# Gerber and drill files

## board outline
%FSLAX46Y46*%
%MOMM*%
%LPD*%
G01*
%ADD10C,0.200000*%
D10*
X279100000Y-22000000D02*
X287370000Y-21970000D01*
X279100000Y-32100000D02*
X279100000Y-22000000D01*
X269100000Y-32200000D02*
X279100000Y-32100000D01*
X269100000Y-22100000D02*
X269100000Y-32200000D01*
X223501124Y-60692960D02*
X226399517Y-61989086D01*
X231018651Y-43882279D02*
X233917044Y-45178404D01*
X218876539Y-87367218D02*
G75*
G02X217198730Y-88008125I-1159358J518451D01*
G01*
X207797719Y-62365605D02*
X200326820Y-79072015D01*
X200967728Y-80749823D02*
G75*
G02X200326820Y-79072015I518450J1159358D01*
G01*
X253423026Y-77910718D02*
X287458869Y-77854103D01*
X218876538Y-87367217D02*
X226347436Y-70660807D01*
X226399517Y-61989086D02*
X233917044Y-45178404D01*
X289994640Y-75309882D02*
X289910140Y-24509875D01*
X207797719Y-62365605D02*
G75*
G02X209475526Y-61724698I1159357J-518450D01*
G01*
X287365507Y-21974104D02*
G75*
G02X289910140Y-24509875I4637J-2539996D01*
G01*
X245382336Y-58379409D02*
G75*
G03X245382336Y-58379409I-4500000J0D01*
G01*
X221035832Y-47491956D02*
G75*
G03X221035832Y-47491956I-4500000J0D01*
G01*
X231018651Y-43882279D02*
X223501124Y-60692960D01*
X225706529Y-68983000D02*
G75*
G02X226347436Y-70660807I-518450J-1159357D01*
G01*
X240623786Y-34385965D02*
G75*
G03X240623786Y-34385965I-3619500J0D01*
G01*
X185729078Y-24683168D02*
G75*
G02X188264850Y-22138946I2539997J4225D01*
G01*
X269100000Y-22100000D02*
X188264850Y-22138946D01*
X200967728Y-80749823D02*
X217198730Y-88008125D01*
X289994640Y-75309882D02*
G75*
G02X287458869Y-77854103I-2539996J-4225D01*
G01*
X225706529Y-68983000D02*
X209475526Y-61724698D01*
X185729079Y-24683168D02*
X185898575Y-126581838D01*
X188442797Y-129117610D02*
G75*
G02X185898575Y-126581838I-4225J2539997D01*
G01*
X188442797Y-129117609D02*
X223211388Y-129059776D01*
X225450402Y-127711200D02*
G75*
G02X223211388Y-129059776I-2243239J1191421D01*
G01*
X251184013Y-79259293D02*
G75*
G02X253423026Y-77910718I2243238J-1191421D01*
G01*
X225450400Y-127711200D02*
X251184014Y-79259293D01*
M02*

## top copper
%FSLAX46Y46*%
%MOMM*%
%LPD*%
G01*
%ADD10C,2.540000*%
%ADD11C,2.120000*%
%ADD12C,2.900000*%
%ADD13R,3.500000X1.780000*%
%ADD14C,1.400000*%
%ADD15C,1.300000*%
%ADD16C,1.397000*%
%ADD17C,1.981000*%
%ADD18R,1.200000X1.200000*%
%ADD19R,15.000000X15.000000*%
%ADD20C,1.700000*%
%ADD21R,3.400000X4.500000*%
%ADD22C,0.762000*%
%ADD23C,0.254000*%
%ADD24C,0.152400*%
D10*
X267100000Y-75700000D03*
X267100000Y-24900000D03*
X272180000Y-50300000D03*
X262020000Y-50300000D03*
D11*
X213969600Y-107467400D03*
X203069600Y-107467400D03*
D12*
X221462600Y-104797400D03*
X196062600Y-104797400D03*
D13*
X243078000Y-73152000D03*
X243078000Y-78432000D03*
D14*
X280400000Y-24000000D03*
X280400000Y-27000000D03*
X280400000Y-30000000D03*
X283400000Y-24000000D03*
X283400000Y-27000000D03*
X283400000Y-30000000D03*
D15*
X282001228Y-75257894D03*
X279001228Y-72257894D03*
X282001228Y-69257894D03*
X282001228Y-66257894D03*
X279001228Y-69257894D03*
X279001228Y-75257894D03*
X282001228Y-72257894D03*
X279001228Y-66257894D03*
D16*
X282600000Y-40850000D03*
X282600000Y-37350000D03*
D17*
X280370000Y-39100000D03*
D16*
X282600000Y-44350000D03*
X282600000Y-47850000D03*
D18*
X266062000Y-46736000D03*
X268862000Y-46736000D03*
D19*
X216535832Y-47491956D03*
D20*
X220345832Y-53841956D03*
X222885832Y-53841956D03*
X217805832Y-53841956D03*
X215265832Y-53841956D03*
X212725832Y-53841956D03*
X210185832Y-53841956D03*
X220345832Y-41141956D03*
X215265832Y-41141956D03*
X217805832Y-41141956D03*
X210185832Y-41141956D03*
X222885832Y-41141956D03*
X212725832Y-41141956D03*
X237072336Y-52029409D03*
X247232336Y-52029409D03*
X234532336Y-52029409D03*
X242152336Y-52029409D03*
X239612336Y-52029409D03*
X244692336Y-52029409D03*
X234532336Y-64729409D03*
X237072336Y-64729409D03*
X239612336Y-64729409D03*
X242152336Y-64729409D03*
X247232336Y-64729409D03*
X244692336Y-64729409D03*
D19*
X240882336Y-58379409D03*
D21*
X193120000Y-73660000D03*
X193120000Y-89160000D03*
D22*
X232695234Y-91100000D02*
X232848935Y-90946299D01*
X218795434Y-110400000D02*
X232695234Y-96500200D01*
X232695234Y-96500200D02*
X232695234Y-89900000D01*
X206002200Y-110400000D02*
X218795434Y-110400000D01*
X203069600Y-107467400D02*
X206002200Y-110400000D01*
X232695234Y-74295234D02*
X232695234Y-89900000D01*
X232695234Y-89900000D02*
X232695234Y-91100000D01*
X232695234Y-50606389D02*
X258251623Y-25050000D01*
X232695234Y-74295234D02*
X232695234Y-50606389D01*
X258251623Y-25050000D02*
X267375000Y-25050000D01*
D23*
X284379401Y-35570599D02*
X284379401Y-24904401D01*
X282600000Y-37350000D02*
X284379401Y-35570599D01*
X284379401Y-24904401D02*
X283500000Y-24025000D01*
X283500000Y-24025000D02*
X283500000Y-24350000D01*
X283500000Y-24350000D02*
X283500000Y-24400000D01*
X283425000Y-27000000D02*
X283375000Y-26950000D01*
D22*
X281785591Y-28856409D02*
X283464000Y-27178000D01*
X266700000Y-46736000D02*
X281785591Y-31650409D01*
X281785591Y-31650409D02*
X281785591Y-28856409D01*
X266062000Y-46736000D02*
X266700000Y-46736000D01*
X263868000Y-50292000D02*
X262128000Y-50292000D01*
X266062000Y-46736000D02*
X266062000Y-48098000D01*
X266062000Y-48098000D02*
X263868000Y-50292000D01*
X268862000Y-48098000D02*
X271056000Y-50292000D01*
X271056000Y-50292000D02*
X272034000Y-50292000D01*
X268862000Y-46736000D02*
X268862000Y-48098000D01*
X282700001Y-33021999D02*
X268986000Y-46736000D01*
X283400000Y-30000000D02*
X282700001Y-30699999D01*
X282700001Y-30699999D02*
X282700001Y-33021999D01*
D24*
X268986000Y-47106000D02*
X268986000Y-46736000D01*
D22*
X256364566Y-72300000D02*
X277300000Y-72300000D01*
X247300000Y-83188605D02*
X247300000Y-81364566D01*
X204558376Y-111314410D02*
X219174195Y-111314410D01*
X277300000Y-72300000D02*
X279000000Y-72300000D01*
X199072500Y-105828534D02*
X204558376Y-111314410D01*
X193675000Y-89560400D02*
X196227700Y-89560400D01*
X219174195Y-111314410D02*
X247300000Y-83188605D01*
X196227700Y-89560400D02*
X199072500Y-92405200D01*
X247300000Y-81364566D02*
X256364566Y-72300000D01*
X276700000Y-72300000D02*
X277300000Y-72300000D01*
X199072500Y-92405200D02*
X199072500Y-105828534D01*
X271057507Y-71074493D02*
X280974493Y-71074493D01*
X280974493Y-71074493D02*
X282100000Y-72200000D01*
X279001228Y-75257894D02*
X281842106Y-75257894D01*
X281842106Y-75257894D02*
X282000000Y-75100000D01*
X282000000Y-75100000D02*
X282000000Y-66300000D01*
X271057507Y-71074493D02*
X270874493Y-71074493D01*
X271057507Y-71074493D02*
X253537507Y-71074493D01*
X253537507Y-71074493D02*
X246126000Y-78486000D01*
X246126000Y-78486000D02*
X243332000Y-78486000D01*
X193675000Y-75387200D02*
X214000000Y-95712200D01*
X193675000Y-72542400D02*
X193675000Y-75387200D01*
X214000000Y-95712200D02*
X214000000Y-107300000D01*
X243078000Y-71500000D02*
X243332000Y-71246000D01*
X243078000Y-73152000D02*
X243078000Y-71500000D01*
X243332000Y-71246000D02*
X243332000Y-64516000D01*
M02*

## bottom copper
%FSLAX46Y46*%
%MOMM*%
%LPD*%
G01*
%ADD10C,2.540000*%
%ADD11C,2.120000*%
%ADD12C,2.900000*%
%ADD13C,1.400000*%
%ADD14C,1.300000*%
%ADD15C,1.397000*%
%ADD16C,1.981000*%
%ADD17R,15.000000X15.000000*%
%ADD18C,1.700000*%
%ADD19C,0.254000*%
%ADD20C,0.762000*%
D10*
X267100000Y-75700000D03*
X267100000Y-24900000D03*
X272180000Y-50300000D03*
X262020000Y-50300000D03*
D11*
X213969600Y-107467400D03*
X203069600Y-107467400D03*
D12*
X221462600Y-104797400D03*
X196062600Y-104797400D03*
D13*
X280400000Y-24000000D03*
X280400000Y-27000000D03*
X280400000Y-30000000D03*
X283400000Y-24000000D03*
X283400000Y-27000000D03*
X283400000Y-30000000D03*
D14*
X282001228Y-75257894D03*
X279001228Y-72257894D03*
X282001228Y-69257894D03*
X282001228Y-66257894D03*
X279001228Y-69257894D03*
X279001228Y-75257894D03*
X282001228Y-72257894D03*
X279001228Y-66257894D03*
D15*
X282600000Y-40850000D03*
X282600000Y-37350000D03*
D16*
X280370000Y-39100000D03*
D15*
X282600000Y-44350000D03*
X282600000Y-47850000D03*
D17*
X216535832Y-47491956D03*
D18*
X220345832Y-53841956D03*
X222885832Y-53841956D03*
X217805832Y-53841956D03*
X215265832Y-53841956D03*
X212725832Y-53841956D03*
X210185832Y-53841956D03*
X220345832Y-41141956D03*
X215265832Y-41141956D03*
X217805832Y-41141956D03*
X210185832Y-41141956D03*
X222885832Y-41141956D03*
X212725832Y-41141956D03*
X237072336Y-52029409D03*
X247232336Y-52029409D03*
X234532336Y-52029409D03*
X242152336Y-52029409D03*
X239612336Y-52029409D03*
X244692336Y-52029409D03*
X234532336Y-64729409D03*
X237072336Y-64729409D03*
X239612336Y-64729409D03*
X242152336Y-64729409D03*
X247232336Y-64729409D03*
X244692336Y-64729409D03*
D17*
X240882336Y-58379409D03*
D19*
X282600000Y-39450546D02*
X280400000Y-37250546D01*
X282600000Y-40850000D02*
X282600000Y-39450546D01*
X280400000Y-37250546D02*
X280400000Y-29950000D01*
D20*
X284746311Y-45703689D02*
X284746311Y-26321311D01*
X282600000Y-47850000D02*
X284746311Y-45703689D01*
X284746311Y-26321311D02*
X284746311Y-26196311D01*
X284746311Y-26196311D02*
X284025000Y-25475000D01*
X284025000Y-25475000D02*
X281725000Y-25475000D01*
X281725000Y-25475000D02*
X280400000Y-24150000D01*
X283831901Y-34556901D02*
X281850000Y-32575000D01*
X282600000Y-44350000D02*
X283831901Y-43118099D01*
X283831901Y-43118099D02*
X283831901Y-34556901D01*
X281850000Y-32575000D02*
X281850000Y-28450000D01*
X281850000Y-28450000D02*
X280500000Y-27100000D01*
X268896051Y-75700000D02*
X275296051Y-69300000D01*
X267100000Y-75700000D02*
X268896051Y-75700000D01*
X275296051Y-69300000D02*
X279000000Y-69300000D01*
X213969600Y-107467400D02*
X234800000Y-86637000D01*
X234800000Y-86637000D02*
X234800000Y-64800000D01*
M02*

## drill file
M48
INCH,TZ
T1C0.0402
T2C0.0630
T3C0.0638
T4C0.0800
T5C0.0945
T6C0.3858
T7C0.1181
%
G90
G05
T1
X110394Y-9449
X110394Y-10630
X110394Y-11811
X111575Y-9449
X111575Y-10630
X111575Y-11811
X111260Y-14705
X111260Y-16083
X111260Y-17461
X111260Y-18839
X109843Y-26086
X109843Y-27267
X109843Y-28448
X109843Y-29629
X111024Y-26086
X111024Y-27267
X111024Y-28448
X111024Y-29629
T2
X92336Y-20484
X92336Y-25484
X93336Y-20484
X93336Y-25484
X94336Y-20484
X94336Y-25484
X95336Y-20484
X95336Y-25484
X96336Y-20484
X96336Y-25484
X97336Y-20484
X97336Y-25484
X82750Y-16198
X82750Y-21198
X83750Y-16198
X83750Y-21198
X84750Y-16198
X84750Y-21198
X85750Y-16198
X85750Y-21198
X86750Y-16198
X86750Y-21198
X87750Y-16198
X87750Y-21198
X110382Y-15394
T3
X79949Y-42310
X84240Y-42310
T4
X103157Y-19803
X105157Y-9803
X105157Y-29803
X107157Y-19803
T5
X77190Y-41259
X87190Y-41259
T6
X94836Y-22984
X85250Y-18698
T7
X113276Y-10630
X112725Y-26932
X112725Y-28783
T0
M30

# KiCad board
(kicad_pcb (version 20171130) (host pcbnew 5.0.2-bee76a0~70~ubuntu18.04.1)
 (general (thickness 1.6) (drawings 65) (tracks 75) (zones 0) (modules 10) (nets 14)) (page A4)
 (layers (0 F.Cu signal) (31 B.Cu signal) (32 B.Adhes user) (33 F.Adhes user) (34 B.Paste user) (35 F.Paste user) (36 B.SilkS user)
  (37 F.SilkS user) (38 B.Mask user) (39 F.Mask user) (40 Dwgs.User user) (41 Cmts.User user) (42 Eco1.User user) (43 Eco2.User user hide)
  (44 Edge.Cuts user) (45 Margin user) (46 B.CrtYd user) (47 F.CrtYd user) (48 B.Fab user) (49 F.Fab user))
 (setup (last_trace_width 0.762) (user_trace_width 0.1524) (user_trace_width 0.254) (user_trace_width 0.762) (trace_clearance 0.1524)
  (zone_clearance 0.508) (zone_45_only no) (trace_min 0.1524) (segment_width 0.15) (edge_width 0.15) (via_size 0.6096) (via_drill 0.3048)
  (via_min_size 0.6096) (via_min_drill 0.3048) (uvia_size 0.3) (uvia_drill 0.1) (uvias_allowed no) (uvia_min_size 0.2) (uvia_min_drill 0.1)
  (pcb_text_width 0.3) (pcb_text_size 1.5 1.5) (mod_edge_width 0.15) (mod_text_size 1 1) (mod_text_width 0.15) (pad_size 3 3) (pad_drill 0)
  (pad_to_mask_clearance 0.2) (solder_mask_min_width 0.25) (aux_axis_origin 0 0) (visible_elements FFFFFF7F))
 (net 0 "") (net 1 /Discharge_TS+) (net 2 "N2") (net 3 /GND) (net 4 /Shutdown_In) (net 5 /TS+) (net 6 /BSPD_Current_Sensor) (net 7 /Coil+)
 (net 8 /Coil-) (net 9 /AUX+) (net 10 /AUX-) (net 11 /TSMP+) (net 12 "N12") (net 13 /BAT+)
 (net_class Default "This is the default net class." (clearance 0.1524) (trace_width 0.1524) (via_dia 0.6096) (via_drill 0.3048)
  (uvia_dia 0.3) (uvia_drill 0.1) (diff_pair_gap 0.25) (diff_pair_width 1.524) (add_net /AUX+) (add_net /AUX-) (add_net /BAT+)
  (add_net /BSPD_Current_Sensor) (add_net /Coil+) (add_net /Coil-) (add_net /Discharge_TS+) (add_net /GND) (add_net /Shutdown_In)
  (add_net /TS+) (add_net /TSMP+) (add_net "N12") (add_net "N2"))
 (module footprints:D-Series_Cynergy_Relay (layer B.Cu) (at 267.1 75.7 90)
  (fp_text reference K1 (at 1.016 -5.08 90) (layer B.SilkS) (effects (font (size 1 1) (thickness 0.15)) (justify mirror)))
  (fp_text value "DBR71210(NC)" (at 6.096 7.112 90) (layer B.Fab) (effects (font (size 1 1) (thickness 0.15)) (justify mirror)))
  (pad 1 thru_hole circle (at 0 0 90) (size 2.54 2.54) (drill 2.032) (layers *.Cu *.Mask) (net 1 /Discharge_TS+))
  (pad 2 thru_hole circle (at 50.8 0 90) (size 2.54 2.54) (drill 2.032) (layers *.Cu *.Mask) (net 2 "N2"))
  (pad 3 thru_hole circle (at 25.4 5.08 90) (size 2.54 2.54) (drill 2.032) (layers *.Cu *.Mask) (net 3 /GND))
  (pad 4 thru_hole circle (at 25.4 -5.08 90) (size 2.54 2.54) (drill 2.032) (layers *.Cu *.Mask) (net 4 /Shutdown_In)))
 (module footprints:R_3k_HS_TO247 (layer B.Cu) (at 213.9696 107.4674 180)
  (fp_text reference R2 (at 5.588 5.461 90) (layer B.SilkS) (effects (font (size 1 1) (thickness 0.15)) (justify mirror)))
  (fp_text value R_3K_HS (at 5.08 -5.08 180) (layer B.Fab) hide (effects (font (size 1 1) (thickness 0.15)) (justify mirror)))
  (pad 1 thru_hole circle (at 0 0 180) (size 2.12 2.12) (drill 1.62) (layers *.Cu *.Mask) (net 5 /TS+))
  (pad 2 thru_hole circle (at 10.9 0 180) (size 2.12 2.12) (drill 1.62) (layers *.Cu *.Mask) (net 2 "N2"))
  (pad 4 thru_hole circle (at -7.493 2.67 180) (size 2.9 2.9) (drill 2.4) (layers *.Cu *.Mask))
  (pad 5 thru_hole circle (at 17.907 2.67 180) (size 2.9 2.9) (drill 2.4) (layers *.Cu *.Mask)))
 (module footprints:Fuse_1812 (layer F.Cu) (at 243.078 73.152 270)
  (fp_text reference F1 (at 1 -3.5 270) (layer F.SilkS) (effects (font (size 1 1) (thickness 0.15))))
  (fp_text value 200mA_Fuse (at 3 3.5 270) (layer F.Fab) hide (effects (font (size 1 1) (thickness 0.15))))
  (pad 1 smd rect (at 0 0 270) (size 1.78 3.5) (layers F.Cu F.Paste F.Mask) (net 5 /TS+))
  (pad 2 smd rect (at 5.28 0 270) (size 1.78 3.5) (layers F.Cu F.Paste F.Mask) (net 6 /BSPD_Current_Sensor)))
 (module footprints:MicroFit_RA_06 (layer B.Cu) (at 287.72 27 90)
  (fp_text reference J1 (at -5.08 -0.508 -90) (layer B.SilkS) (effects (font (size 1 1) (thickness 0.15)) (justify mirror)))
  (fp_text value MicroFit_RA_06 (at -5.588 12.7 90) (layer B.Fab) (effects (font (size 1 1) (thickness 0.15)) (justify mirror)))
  (pad 6 thru_hole circle (at 3 -7.32 270) (size 1.4 1.4) (drill 1.02) (layers *.Cu *.Mask) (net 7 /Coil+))
  (pad 5 thru_hole circle (at 0 -7.32 270) (size 1.4 1.4) (drill 1.02) (layers *.Cu *.Mask) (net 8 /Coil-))
  (pad 4 thru_hole circle (at -3 -7.32 270) (size 1.4 1.4) (drill 1.02) (layers *.Cu *.Mask) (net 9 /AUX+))
  (pad 3 thru_hole circle (at 3 -4.32 270) (size 1.4 1.4) (drill 1.02) (layers *.Cu *.Mask) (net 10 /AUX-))
  (pad 2 thru_hole circle (at 0 -4.32 270) (size 1.4 1.4) (drill 1.02) (layers *.Cu *.Mask) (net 4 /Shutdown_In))
  (pad 1 thru_hole circle (at -3 -4.32 270) (size 1.4 1.4) (drill 1.02) (layers *.Cu *.Mask) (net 3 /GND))
  (pad "" np_thru_hole circle (at 0 0 270) (size 3 3) (drill 3) (layers *.Cu *.Mask)))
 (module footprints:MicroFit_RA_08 (layer B.Cu) (at 286.4104 70.6374 90)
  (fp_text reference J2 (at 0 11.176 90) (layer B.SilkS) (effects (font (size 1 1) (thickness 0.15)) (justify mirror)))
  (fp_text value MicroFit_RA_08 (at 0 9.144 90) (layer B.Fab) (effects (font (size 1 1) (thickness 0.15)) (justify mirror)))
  (pad "" np_thru_hole circle (at -2.470494 -0.089172 270) (size 3 3) (drill 3) (layers *.Cu *.Mask))
  (pad "" np_thru_hole circle (at 2.229506 -0.089172 270) (size 3 3) (drill 3) (layers *.Cu *.Mask))
  (pad 1 thru_hole circle (at -4.620494 -4.409172 270) (size 1.3 1.3) (drill 1.02) (layers *.Cu *.Mask) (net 6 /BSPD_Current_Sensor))
  (pad 6 thru_hole circle (at -1.620494 -7.409172 270) (size 1.3 1.3) (drill 1.02) (layers *.Cu *.Mask) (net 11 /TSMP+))
  (pad 3 thru_hole circle (at 1.379506 -4.409172 270) (size 1.3 1.3) (drill 1.02) (layers *.Cu *.Mask) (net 6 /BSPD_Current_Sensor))
  (pad 4 thru_hole circle (at 4.379506 -4.409172 270) (size 1.3 1.3) (drill 1.02) (layers *.Cu *.Mask) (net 6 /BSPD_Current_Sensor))
  (pad 7 thru_hole circle (at 1.379506 -7.409172 270) (size 1.3 1.3) (drill 1.02) (layers *.Cu *.Mask) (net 1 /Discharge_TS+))
  (pad 5 thru_hole circle (at -4.620494 -7.409172 270) (size 1.3 1.3) (drill 1.02) (layers *.Cu *.Mask) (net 6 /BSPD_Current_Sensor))
  (pad 2 thru_hole circle (at -1.620494 -4.409172 270) (size 1.3 1.3) (drill 1.02) (layers *.Cu *.Mask) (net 6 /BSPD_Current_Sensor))
  (pad 8 thru_hole circle (at 4.379506 -7.409172 270) (size 1.3 1.3) (drill 1.02) (layers *.Cu *.Mask) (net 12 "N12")))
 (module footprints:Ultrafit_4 (layer F.Cu) (at 282.6 42.6 180)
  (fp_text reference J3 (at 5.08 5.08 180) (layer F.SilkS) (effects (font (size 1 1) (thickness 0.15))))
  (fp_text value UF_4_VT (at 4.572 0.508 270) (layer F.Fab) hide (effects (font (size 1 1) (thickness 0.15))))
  (pad 2 thru_hole circle (at 0 1.75 180) (size 1.397 1.397) (drill 1.02) (layers *.Cu *.Mask) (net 9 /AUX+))
  (pad 1 thru_hole circle (at 0 5.25 180) (size 1.397 1.397) (drill 1.02) (layers *.Cu *.Mask) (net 10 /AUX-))
  (pad "" thru_hole circle (at 2.23 3.5 180) (size 1.981 1.981) (drill 1.6) (layers *.Cu *.Mask))
  (pad 3 thru_hole circle (at 0 -1.75) (size 1.397 1.397) (drill 1.02) (layers *.Cu *.Mask) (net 8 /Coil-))
  (pad 4 thru_hole circle (at 0 -5.25) (size 1.397 1.397) (drill 1.02) (layers *.Cu *.Mask) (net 7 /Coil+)))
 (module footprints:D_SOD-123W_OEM (layer F.Cu) (at 267.462 46.736)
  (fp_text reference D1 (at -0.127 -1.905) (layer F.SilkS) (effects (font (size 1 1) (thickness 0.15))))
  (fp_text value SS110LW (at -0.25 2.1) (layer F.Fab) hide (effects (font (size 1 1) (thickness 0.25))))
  (pad 1 smd rect (at -1.4 0) (size 1.2 1.2) (layers F.Cu F.Paste F.Mask) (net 4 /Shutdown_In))
  (pad 2 smd rect (at 1.4 0) (size 1.2 1.2) (layers F.Cu F.Paste F.Mask) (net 3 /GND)))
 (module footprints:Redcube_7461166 (layer F.Cu) (at 216.535832 47.491956)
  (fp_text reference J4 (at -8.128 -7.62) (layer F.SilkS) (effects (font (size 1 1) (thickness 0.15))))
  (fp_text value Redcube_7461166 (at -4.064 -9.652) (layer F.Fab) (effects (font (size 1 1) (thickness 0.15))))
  (pad 1 thru_hole rect (at 0 0) (size 15 15) (drill 9.8) (layers *.Cu *.Mask) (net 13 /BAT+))
  (pad 1 thru_hole circle (at 3.81 6.35) (size 1.7 1.7) (drill 1.6) (layers *.Cu *.Mask) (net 13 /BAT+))
  (pad 1 thru_hole circle (at 6.35 6.35) (size 1.7 1.7) (drill 1.6) (layers *.Cu *.Mask) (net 13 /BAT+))
  (pad 1 thru_hole circle (at 1.27 6.35) (size 1.7 1.7) (drill 1.6) (layers *.Cu *.Mask) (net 13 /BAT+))
  (pad 1 thru_hole circle (at -1.27 6.35) (size 1.7 1.7) (drill 1.6) (layers *.Cu *.Mask) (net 13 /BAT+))
  (pad 1 thru_hole circle (at -3.81 6.35) (size 1.7 1.7) (drill 1.6) (layers *.Cu *.Mask) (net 13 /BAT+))
  (pad 1 thru_hole circle (at -6.35 6.35) (size 1.7 1.7) (drill 1.6) (layers *.Cu *.Mask) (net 13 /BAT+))
  (pad 1 thru_hole circle (at 3.81 -6.35) (size 1.7 1.7) (drill 1.6) (layers *.Cu *.Mask) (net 13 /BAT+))
  (pad 1 thru_hole circle (at -1.27 -6.35) (size 1.7 1.7) (drill 1.6) (layers *.Cu *.Mask) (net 13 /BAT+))
  (pad 1 thru_hole circle (at 1.27 -6.35) (size 1.7 1.7) (drill 1.6) (layers *.Cu *.Mask) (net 13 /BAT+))
  (pad 1 thru_hole circle (at -6.35 -6.35) (size 1.7 1.7) (drill 1.6) (layers *.Cu *.Mask) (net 13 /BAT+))
  (pad 1 thru_hole circle (at 6.35 -6.35) (size 1.7 1.7) (drill 1.6) (layers *.Cu *.Mask) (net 13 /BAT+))
  (pad 1 thru_hole circle (at -3.81 -6.35) (size 1.7 1.7) (drill 1.6) (layers *.Cu *.Mask) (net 13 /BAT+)))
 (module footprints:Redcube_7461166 (layer F.Cu) (at 240.882336 58.379409)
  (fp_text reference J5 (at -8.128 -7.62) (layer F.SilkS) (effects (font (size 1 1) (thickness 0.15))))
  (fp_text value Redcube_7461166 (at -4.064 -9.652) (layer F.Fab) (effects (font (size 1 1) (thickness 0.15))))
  (pad 1 thru_hole circle (at -3.81 -6.35) (size 1.7 1.7) (drill 1.6) (layers *.Cu *.Mask) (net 5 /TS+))
  (pad 1 thru_hole circle (at 6.35 -6.35) (size 1.7 1.7) (drill 1.6) (layers *.Cu *.Mask) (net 5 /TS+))
  (pad 1 thru_hole circle (at -6.35 -6.35) (size 1.7 1.7) (drill 1.6) (layers *.Cu *.Mask) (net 5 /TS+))
  (pad 1 thru_hole circle (at 1.27 -6.35) (size 1.7 1.7) (drill 1.6) (layers *.Cu *.Mask) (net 5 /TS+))
  (pad 1 thru_hole circle (at -1.27 -6.35) (size 1.7 1.7) (drill 1.6) (layers *.Cu *.Mask) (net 5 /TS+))
  (pad 1 thru_hole circle (at 3.81 -6.35) (size 1.7 1.7) (drill 1.6) (layers *.Cu *.Mask) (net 5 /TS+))
  (pad 1 thru_hole circle (at -6.35 6.35) (size 1.7 1.7) (drill 1.6) (layers *.Cu *.Mask) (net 5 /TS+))
  (pad 1 thru_hole circle (at -3.81 6.35) (size 1.7 1.7) (drill 1.6) (layers *.Cu *.Mask) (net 5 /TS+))
  (pad 1 thru_hole circle (at -1.27 6.35) (size 1.7 1.7) (drill 1.6) (layers *.Cu *.Mask) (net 5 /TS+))
  (pad 1 thru_hole circle (at 1.27 6.35) (size 1.7 1.7) (drill 1.6) (layers *.Cu *.Mask) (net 5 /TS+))
  (pad 1 thru_hole circle (at 6.35 6.35) (size 1.7 1.7) (drill 1.6) (layers *.Cu *.Mask) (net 5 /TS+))
  (pad 1 thru_hole circle (at 3.81 6.35) (size 1.7 1.7) (drill 1.6) (layers *.Cu *.Mask) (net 5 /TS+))
  (pad 1 thru_hole rect (at 0 0) (size 15 15) (drill 9.8) (layers *.Cu *.Mask) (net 5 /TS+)))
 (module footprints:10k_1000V (layer F.Cu) (at 193.12 73.66 270)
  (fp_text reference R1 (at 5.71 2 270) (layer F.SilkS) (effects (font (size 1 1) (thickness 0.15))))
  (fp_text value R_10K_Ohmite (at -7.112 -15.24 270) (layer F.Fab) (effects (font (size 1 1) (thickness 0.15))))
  (pad 1 smd rect (at 0 0 270) (size 4.5 3.4) (layers F.Cu F.Paste F.Mask) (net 5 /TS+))
  (pad 2 smd rect (at 15.5 0 270) (size 4.5 3.4) (layers F.Cu F.Paste F.Mask) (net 11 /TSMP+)))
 (gr_line (start 279.1 22) (end 287.37 21.97) (layer Edge.Cuts) (width 0.2))
 (gr_line (start 279.1 32.1) (end 279.1 22) (layer Edge.Cuts) (width 0.2))
 (gr_line (start 269.1 32.2) (end 279.1 32.1) (layer Edge.Cuts) (width 0.2))
 (gr_line (start 269.1 22.1) (end 269.1 32.2) (layer Edge.Cuts) (width 0.2))
 (gr_line (start 223.501124 60.69296) (end 226.399517 61.989086) (layer Edge.Cuts) (width 0.2))
 (gr_line (start 231.018651 43.882279) (end 233.917044 45.178404) (layer Edge.Cuts) (width 0.2))
 (gr_arc (start 217.717181 86.848767) (end 217.19873 88.008125) (angle -90) (layer Edge.Cuts) (width 0.2))
 (gr_line (start 207.797719 62.365605) (end 200.32682 79.072015) (layer Edge.Cuts) (width 0.2))
 (gr_arc (start 201.486178 79.590465) (end 200.32682 79.072015) (angle -90) (layer Edge.Cuts) (width 0.2))
 (gr_line (start 253.423026 77.910718) (end 287.458869 77.854103) (layer Edge.Cuts) (width 0.2))
 (gr_line (start 218.876538 87.367217) (end 226.347436 70.660807) (layer Edge.Cuts) (width 0.2))
 (gr_line (start 226.399517 61.989086) (end 233.917044 45.178404) (layer Edge.Cuts) (width 0.2))
 (gr_line (start 289.99464 75.309882) (end 289.91014 24.509875) (layer Edge.Cuts) (width 0.2))
 (gr_arc (start 208.957076 62.884055) (end 209.475526 61.724698) (angle -90) (layer Edge.Cuts) (width 0.2))
 (gr_arc (start 287.370144 24.5141) (end 289.91014 24.509875) (angle -90.00930339) (layer Edge.Cuts) (width 0.2))
 (gr_circle (center 240.882336 58.379409) (end 245.382336 58.379409) (layer Edge.Cuts) (width 0.2))
 (gr_circle (center 216.535832 47.491956) (end 221.035832 47.491956) (layer Edge.Cuts) (width 0.2))
 (gr_line (start 231.018651 43.882279) (end 223.501124 60.69296) (layer Edge.Cuts) (width 0.2))
 (gr_arc (start 225.188079 70.142357) (end 226.347436 70.660807) (angle -90) (layer Edge.Cuts) (width 0.2))
 (gr_circle (center 237.004286 34.385965) (end 240.623786 34.385965) (layer Edge.Cuts) (width 0.2))
 (gr_arc (start 188.269075 24.678943) (end 188.26485 22.138946) (angle -90) (layer Edge.Cuts) (width 0.2))
 (gr_line (start 269.1 22.1) (end 188.26485 22.138946) (layer Edge.Cuts) (width 0.2))
 (gr_line (start 200.967728 80.749823) (end 217.19873 88.008125) (layer Edge.Cuts) (width 0.2))
 (gr_arc (start 287.454644 75.314107) (end 287.458869 77.854103) (angle -90) (layer Edge.Cuts) (width 0.2))
 (gr_line (start 225.706529 68.983) (end 209.475526 61.724698) (layer Edge.Cuts) (width 0.2))
 (gr_line (start 185.729079 24.683168) (end 185.898575 126.581838) (layer Edge.Cuts) (width 0.2))
 (gr_arc (start 188.438572 126.577613) (end 185.898575 126.581838) (angle -90) (layer Edge.Cuts) (width 0.2))
 (gr_line (start 188.442797 129.117609) (end 223.211388 129.059776) (layer Edge.Cuts) (width 0.2))
 (gr_arc (start 223.207163 126.519779) (end 223.211388 129.059776) (angle -61.93118106) (layer Edge.Cuts) (width 0.2))
 (gr_arc (start 253.427251 80.450714) (end 253.423026 77.910718) (angle -61.93118106) (layer Edge.Cuts) (width 0.2))
 (gr_line (start 225.4504 127.7112) (end 251.184014 79.259293) (layer Edge.Cuts) (width 0.2))
 (segment (start 232.695234 91.1) (end 232.848935 90.946299) (width 0.762) (layer F.Cu) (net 2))
 (segment (start 218.795434 110.4) (end 232.695234 96.5002) (width 0.762) (layer F.Cu) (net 2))
 (segment (start 232.695234 96.5002) (end 232.695234 89.9) (width 0.762) (layer F.Cu) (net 2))
 (segment (start 206.0022 110.4) (end 218.795434 110.4) (width 0.762) (layer F.Cu) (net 2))
 (segment (start 203.0696 107.4674) (end 206.0022 110.4) (width 0.762) (layer F.Cu) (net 2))
 (segment (start 232.695234 74.295234) (end 232.695234 89.9) (width 0.762) (layer F.Cu) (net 2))
 (segment (start 232.695234 89.9) (end 232.695234 91.1) (width 0.762) (layer F.Cu) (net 2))
 (segment (start 232.695234 50.606389) (end 258.251623 25.05) (width 0.762) (layer F.Cu) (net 2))
 (segment (start 232.695234 74.295234) (end 232.695234 50.606389) (width 0.762) (layer F.Cu) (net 2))
 (segment (start 258.251623 25.05) (end 267.375 25.05) (width 0.762) (layer F.Cu) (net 2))
 (segment (start 282.6 39.450546) (end 280.4 37.250546) (width 0.254) (layer B.Cu) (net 9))
 (segment (start 282.6 40.85) (end 282.6 39.450546) (width 0.254) (layer B.Cu) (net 9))
 (segment (start 280.4 37.250546) (end 280.4 29.95) (width 0.254) (layer B.Cu) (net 9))
 (segment (start 284.379401 35.570599) (end 284.379401 24.904401) (width 0.254) (layer F.Cu) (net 10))
 (segment (start 282.6 37.35) (end 284.379401 35.570599) (width 0.254) (layer F.Cu) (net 10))
 (segment (start 284.379401 24.904401) (end 283.5 24.025) (width 0.254) (layer F.Cu) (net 10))
 (segment (start 283.5 24.025) (end 283.5 24.35) (width 0.254) (layer F.Cu) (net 10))
 (segment (start 283.5 24.35) (end 283.5 24.4) (width 0.254) (layer F.Cu) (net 10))
 (segment (start 284.746311 45.703689) (end 284.746311 26.321311) (width 0.762) (layer B.Cu) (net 7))
 (segment (start 282.6 47.85) (end 284.746311 45.703689) (width 0.762) (layer B.Cu) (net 7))
 (segment (start 284.746311 26.321311) (end 284.746311 26.196311) (width 0.762) (layer B.Cu) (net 7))
 (segment (start 284.746311 26.196311) (end 284.025 25.475) (width 0.762) (layer B.Cu) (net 7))
 (segment (start 284.025 25.475) (end 281.725 25.475) (width 0.762) (layer B.Cu) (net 7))
 (segment (start 281.725 25.475) (end 280.4 24.15) (width 0.762) (layer B.Cu) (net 7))
 (segment (start 283.831901 34.556901) (end 281.85 32.575) (width 0.762) (layer B.Cu) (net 8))
 (segment (start 282.6 44.35) (end 283.831901 43.118099) (width 0.762) (layer B.Cu) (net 8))
 (segment (start 283.831901 43.118099) (end 283.831901 34.556901) (width 0.762) (layer B.Cu) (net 8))
 (segment (start 281.85 32.575) (end 281.85 28.45) (width 0.762) (layer B.Cu) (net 8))
 (segment (start 281.85 28.45) (end 280.5 27.1) (width 0.762) (layer B.Cu) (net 8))
 (segment (start 283.425 27) (end 283.375 26.95) (width 0.254) (layer F.Cu) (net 4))
 (segment (start 281.785591 28.856409) (end 283.464 27.178) (width 0.762) (layer F.Cu) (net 4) (status 1000000))
 (segment (start 266.7 46.736) (end 281.785591 31.650409) (width 0.762) (layer F.Cu) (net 4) (status 1000000))
 (segment (start 281.785591 31.650409) (end 281.785591 28.856409) (width 0.762) (layer F.Cu) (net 4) (status 1000000))
 (segment (start 266.062 46.736) (end 266.7 46.736) (width 0.762) (layer F.Cu) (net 4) (status 1000000))
 (segment (start 263.868 50.292) (end 262.128 50.292) (width 0.762) (layer F.Cu) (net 4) (status 1000000))
 (segment (start 266.062 46.736) (end 266.062 48.098) (width 0.762) (layer F.Cu) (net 4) (status 1000000))
 (segment (start 266.062 48.098) (end 263.868 50.292) (width 0.762) (layer F.Cu) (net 4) (status 1000000))
 (segment (start 268.862 48.098) (end 271.056 50.292) (width 0.762) (layer F.Cu) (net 3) (status 1000000))
 (segment (start 271.056 50.292) (end 272.034 50.292) (width 0.762) (layer F.Cu) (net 3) (status 1000000))
 (segment (start 268.862 46.736) (end 268.862 48.098) (width 0.762) (layer F.Cu) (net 3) (status 1000000))
 (segment (start 282.700001 33.021999) (end 268.986 46.736) (width 0.762) (layer F.Cu) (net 3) (status 1000000))
 (segment (start 283.4 30) (end 282.700001 30.699999) (width 0.762) (layer F.Cu) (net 3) (status 1000000))
 (segment (start 282.700001 30.699999) (end 282.700001 33.021999) (width 0.762) (layer F.Cu) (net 3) (status 1000000))
 (segment (start 268.986 47.106) (end 268.986 46.736) (width 0.1524) (layer F.Cu) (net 3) (status 1000000))
 (segment (start 256.364566 72.3) (end 277.3 72.3) (width 0.762) (layer F.Cu) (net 11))
 (segment (start 247.3 83.188605) (end 247.3 81.364566) (width 0.762) (layer F.Cu) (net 11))
 (segment (start 204.558376 111.31441) (end 219.174195 111.31441) (width 0.762) (layer F.Cu) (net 11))
 (segment (start 277.3 72.3) (end 279 72.3) (width 0.762) (layer F.Cu) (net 11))
 (segment (start 199.0725 105.828534) (end 204.558376 111.31441) (width 0.762) (layer F.Cu) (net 11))
 (segment (start 193.675 89.5604) (end 196.2277 89.5604) (width 0.762) (layer F.Cu) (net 11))
 (segment (start 219.174195 111.31441) (end 247.3 83.188605) (width 0.762) (layer F.Cu) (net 11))
 (segment (start 196.2277 89.5604) (end 199.0725 92.4052) (width 0.762) (layer F.Cu) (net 11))
 (segment (start 247.3 81.364566) (end 256.364566 72.3) (width 0.762) (layer F.Cu) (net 11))
 (segment (start 276.7 72.3) (end 277.3 72.3) (width 0.762) (layer F.Cu) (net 11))
 (segment (start 199.0725 92.4052) (end 199.0725 105.828534) (width 0.762) (layer F.Cu) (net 11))
 (segment (start 271.057507 71.074493) (end 280.974493 71.074493) (width 0.762) (layer F.Cu) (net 6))
 (segment (start 280.974493 71.074493) (end 282.1 72.2) (width 0.762) (layer F.Cu) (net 6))
 (segment (start 279.001228 75.257894) (end 281.842106 75.257894) (width 0.762) (layer F.Cu) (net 6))
 (segment (start 281.842106 75.257894) (end 282 75.1) (width 0.762) (layer F.Cu) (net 6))
 (segment (start 282 75.1) (end 282 66.3) (width 0.762) (layer F.Cu) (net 6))
 (segment (start 271.057507 71.074493) (end 270.874493 71.074493) (width 0.762) (layer F.Cu) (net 6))
 (segment (start 271.057507 71.074493) (end 253.537507 71.074493) (width 0.762) (layer F.Cu) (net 6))
 (segment (start 253.537507 71.074493) (end 246.126 78.486) (width 0.762) (layer F.Cu) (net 6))
 (segment (start 246.126 78.486) (end 243.332 78.486) (width 0.762) (layer F.Cu) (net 6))
 (segment (start 268.896051 75.7) (end 275.296051 69.3) (width 0.762) (layer B.Cu) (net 1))
 (segment (start 267.1 75.7) (end 268.896051 75.7) (width 0.762) (layer B.Cu) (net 1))
 (segment (start 275.296051 69.3) (end 279 69.3) (width 0.762) (layer B.Cu) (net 1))
 (segment (start 213.9696 107.4674) (end 234.8 86.637) (width 0.762) (layer B.Cu) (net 5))
 (segment (start 234.8 86.637) (end 234.8 64.8) (width 0.762) (layer B.Cu) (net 5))
 (segment (start 193.675 75.3872) (end 214 95.7122) (width 0.762) (layer F.Cu) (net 5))
 (segment (start 193.675 72.5424) (end 193.675 75.3872) (width 0.762) (layer F.Cu) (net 5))
 (segment (start 214 95.7122) (end 214 107.3) (width 0.762) (layer F.Cu) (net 5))
 (segment (start 243.078 71.5) (end 243.332 71.246) (width 0.762) (layer F.Cu) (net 5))
 (segment (start 243.078 73.152) (end 243.078 71.5) (width 0.762) (layer F.Cu) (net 5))
 (segment (start 243.332 71.246) (end 243.332 64.516) (width 0.762) (layer F.Cu) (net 5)))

